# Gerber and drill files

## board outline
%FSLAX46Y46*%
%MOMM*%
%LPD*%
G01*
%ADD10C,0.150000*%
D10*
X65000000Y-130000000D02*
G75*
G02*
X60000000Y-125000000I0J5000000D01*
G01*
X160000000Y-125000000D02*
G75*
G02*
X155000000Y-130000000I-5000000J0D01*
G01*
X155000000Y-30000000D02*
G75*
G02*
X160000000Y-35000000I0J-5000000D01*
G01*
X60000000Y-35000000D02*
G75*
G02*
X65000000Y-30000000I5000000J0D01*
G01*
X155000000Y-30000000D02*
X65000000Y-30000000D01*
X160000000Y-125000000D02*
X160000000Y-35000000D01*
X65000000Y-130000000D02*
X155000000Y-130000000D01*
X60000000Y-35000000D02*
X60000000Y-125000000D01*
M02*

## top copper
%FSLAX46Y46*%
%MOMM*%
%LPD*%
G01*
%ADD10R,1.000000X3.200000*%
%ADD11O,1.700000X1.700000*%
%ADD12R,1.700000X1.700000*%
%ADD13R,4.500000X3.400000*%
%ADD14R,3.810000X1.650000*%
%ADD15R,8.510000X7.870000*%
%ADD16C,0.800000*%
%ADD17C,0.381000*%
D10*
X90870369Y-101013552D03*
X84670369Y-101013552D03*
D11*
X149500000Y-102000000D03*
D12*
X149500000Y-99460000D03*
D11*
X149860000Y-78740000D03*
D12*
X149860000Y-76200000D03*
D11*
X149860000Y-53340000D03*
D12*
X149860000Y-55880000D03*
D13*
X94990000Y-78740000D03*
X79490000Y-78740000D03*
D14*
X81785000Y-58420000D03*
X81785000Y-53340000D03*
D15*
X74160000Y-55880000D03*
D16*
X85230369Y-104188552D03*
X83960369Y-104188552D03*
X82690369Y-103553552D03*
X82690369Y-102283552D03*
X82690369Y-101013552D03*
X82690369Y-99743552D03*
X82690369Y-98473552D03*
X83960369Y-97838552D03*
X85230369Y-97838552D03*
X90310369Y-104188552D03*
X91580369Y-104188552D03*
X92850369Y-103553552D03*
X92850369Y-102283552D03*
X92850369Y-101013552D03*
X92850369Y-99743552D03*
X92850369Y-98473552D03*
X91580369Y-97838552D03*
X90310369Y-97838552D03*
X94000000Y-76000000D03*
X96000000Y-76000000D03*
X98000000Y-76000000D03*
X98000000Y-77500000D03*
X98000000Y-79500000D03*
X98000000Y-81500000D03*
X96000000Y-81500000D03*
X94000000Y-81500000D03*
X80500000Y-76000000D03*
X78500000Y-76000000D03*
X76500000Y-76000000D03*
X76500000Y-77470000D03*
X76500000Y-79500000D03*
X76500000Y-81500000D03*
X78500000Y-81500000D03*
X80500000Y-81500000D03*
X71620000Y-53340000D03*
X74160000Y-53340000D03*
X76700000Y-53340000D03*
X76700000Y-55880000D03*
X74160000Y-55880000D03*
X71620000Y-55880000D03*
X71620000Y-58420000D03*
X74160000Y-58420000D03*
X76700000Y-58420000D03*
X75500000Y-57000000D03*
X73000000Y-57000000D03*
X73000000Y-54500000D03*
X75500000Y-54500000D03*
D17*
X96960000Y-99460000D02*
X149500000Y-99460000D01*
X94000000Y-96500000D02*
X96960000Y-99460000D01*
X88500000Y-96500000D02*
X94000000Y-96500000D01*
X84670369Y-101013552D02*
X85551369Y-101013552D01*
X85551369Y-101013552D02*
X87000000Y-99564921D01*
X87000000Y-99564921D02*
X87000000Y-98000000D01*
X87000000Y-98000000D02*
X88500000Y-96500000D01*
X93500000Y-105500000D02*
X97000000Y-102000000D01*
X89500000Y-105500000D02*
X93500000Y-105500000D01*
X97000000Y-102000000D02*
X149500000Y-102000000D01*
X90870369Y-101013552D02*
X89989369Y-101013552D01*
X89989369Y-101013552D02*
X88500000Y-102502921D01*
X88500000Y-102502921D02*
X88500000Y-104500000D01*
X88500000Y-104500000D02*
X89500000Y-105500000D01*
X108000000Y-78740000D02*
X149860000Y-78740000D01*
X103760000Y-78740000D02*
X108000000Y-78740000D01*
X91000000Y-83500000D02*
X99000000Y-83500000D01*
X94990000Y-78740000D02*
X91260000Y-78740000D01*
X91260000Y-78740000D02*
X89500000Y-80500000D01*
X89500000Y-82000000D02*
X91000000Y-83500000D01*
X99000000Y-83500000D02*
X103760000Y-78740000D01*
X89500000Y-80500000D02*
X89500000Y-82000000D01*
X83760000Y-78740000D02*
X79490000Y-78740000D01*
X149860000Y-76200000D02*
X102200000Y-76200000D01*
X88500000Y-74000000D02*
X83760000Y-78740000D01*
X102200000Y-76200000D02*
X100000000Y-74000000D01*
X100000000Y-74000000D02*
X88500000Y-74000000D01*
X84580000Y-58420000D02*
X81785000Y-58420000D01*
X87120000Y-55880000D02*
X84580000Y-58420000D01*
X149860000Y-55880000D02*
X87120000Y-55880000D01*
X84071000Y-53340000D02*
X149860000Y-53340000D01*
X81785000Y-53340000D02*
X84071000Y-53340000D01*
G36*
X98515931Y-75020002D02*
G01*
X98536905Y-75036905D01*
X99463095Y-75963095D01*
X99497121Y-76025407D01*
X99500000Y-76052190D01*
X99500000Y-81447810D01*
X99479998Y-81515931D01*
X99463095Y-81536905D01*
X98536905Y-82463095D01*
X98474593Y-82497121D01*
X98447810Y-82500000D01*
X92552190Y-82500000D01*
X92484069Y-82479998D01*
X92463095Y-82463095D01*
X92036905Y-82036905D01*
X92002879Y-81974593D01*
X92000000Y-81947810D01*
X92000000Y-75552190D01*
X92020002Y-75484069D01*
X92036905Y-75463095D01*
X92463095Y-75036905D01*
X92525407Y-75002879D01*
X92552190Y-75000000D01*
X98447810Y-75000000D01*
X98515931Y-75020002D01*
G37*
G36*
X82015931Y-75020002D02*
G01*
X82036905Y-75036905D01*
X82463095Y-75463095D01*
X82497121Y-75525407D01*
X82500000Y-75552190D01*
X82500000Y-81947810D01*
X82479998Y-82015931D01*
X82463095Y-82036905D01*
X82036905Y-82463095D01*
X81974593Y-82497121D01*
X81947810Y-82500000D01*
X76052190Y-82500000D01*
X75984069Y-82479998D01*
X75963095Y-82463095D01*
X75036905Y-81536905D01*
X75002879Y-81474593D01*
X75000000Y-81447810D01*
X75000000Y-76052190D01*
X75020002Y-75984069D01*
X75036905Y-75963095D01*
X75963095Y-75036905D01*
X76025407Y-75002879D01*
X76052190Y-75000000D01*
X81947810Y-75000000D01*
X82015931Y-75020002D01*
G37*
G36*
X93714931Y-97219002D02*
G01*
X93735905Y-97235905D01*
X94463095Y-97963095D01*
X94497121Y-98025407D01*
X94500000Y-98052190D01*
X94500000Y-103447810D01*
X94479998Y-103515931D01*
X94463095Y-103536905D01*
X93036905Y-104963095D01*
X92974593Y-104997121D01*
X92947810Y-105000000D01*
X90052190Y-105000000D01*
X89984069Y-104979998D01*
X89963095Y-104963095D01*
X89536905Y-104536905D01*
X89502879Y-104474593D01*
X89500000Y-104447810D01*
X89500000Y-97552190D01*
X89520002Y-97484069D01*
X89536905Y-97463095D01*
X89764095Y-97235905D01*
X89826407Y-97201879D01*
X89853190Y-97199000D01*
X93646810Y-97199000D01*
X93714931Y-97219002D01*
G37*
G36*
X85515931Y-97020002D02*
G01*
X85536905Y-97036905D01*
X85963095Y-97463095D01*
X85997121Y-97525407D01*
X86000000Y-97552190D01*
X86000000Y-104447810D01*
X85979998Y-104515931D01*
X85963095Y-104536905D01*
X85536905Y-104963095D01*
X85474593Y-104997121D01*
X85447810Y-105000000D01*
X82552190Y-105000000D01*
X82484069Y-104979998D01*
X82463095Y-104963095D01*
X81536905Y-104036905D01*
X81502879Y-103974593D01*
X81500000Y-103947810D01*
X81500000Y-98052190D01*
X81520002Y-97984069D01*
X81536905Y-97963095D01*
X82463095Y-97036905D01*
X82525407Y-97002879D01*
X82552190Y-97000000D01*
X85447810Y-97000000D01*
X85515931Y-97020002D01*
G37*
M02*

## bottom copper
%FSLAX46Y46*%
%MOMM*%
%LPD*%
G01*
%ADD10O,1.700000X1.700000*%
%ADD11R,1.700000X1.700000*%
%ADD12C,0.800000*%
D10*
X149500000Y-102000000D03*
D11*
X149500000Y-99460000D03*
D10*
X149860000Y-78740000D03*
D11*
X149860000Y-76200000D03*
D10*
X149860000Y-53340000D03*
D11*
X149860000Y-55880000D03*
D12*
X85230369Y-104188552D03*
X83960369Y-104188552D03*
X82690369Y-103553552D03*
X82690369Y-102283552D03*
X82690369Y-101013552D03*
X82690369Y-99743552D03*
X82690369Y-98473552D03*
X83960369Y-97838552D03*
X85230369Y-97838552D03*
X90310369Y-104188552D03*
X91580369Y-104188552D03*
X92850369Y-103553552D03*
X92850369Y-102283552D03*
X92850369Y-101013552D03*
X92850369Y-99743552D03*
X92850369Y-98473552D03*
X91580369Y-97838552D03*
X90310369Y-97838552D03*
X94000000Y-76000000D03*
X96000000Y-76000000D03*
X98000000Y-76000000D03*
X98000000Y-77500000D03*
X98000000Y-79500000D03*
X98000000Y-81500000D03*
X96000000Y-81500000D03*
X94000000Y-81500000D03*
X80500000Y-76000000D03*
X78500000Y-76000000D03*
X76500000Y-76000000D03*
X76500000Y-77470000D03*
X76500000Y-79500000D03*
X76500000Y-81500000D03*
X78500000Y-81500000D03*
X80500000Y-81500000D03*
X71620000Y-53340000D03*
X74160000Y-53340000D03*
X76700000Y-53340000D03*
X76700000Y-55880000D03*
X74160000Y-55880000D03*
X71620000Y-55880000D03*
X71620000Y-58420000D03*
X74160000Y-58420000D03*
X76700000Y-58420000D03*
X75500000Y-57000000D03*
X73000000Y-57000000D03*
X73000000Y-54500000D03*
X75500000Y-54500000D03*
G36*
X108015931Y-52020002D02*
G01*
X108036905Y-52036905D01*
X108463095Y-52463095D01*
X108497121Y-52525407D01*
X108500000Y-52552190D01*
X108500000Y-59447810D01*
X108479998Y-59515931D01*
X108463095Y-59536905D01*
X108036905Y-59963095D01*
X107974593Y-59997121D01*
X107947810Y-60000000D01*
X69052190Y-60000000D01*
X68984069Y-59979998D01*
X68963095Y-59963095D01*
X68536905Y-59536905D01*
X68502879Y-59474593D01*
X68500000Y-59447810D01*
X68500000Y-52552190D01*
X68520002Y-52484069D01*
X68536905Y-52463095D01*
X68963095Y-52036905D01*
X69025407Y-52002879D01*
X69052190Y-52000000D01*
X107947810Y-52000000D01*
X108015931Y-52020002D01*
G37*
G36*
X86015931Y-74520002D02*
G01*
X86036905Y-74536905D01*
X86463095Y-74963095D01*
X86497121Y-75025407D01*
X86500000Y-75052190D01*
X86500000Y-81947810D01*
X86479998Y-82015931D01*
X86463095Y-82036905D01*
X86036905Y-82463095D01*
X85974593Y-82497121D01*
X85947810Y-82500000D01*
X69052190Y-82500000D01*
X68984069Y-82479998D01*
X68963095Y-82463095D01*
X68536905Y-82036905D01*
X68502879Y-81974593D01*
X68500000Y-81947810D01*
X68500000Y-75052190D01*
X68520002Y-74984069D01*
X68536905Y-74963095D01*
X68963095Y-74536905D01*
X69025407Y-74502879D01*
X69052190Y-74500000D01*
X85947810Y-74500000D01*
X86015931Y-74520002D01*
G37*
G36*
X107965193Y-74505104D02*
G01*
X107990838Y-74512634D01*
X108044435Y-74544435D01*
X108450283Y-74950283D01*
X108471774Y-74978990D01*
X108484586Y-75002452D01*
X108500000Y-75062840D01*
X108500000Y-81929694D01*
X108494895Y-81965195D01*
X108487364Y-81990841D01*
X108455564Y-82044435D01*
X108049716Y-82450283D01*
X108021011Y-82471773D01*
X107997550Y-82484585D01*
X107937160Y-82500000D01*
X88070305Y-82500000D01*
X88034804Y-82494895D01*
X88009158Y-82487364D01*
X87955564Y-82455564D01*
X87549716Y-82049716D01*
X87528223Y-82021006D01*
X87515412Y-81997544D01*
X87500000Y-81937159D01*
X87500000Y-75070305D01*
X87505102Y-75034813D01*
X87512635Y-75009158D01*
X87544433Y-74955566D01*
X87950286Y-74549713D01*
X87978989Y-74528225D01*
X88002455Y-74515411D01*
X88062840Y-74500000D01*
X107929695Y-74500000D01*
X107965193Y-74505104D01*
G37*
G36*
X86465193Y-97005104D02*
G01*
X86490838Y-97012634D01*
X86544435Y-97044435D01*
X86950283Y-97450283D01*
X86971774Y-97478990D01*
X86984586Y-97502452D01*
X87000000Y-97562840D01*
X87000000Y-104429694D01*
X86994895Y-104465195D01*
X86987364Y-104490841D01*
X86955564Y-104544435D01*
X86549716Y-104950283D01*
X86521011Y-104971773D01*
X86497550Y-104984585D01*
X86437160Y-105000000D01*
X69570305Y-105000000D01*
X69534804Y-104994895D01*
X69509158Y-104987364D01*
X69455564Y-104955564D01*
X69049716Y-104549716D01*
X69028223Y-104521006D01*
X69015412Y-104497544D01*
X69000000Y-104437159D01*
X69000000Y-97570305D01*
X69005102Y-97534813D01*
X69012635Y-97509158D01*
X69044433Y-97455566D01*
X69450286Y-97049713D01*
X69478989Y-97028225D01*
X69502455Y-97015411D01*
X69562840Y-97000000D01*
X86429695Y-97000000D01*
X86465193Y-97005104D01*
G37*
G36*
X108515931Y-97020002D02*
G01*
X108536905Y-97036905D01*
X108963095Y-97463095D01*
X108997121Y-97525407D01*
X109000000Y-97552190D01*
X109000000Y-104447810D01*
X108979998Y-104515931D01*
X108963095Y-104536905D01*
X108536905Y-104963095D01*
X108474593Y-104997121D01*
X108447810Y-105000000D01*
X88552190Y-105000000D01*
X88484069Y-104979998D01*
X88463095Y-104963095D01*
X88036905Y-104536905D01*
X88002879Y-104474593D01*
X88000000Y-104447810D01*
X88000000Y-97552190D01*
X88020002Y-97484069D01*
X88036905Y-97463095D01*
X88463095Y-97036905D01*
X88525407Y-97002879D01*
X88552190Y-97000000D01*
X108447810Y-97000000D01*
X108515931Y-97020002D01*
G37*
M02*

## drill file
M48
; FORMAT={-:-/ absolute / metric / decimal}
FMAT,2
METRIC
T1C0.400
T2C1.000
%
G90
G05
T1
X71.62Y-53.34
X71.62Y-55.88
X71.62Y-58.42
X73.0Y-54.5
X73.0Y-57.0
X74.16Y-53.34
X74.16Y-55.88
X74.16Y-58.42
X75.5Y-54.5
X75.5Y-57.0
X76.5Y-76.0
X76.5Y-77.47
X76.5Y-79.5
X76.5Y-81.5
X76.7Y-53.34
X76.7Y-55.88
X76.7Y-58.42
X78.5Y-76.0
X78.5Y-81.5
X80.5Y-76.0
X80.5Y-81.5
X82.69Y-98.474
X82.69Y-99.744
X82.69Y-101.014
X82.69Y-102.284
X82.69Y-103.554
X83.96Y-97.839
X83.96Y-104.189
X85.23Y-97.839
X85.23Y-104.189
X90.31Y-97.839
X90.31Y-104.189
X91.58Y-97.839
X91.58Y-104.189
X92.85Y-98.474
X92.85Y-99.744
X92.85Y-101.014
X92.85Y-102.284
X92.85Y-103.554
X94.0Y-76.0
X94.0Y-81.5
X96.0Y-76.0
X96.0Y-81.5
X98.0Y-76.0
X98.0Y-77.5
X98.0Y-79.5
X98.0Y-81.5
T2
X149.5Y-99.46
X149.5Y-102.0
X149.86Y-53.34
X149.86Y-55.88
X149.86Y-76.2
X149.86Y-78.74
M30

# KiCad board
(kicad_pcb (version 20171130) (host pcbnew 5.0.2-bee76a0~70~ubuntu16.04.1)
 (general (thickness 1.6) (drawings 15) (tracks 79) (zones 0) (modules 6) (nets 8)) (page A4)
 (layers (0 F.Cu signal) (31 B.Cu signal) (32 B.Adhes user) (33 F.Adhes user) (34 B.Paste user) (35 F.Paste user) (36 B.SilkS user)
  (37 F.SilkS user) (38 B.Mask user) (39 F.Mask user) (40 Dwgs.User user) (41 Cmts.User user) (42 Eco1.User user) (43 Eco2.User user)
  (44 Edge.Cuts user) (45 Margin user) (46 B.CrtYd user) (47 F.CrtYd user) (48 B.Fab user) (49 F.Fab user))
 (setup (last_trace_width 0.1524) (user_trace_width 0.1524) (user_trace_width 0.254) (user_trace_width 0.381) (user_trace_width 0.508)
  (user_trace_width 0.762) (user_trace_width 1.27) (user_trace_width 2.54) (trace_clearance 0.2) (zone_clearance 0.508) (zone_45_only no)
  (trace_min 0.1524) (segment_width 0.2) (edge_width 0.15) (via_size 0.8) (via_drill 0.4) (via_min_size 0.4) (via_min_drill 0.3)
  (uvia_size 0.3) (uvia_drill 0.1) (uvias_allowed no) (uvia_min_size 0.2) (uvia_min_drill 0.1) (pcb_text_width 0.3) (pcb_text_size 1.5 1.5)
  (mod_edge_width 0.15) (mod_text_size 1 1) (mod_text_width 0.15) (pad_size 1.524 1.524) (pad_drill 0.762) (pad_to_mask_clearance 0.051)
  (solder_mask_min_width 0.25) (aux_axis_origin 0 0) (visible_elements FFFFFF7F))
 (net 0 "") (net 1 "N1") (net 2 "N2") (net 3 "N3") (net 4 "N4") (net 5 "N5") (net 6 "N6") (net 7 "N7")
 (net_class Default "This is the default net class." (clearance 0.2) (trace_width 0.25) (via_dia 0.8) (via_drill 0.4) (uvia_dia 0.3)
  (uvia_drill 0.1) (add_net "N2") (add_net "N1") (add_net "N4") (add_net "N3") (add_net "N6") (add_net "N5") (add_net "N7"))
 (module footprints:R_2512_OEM (layer F.Cu) (at 87.770369 101.013552)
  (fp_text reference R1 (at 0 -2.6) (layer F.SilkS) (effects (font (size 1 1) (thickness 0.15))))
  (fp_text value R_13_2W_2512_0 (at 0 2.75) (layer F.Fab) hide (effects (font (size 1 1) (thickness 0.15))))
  (pad 2 smd rect (at 3.1 0) (size 1 3.2) (layers F.Cu F.Paste F.Mask) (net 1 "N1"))
  (pad 1 smd rect (at -3.1 0) (size 1 3.2) (layers F.Cu F.Paste F.Mask) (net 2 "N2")))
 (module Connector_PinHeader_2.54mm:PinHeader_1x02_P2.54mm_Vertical (layer F.Cu) (at 149.5 99.46)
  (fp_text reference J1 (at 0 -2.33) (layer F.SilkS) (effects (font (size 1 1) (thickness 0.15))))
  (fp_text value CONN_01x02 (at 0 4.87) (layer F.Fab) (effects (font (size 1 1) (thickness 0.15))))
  (pad 2 thru_hole oval (at 0 2.54) (size 1.7 1.7) (drill 1) (layers *.Cu *.Mask) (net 1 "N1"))
  (pad 1 thru_hole rect (at 0 0) (size 1.7 1.7) (drill 1) (layers *.Cu *.Mask) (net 2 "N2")))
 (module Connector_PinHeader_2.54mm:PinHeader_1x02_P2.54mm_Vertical (layer F.Cu) (at 149.86 76.2)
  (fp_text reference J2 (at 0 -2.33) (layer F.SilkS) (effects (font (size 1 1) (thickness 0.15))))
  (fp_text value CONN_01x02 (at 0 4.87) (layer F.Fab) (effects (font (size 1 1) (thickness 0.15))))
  (pad 2 thru_hole oval (at 0 2.54) (size 1.7 1.7) (drill 1) (layers *.Cu *.Mask) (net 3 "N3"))
  (pad 1 thru_hole rect (at 0 0) (size 1.7 1.7) (drill 1) (layers *.Cu *.Mask) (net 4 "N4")))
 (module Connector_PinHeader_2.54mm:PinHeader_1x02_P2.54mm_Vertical (layer F.Cu) (at 149.86 55.88 180)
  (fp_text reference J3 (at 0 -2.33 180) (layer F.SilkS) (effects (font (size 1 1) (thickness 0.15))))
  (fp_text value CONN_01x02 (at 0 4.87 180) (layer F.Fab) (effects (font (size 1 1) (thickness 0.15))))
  (pad 2 thru_hole oval (at 0 2.54 180) (size 1.7 1.7) (drill 1) (layers *.Cu *.Mask) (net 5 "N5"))
  (pad 1 thru_hole rect (at 0 0 180) (size 1.7 1.7) (drill 1) (layers *.Cu *.Mask) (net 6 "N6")))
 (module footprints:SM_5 (layer F.Cu) (at 87.24 78.74)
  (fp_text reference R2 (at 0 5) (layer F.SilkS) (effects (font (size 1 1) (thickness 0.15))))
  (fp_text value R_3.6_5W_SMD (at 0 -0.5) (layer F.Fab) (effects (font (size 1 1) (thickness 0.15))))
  (pad 2 smd rect (at 7.75 0) (size 4.5 3.4) (layers F.Cu F.Paste F.Mask) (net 3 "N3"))
  (pad 1 smd rect (at -7.75 0) (size 4.5 3.4) (layers F.Cu F.Paste F.Mask) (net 4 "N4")))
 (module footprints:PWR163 (layer F.Cu) (at 74.16 55.88 90)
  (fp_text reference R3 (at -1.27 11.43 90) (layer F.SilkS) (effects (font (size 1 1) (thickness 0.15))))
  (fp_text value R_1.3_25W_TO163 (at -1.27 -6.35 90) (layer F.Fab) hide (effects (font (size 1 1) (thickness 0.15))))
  (pad 1 smd rect (at -2.54 7.625 90) (size 1.65 3.81) (layers F.Cu F.Paste F.Mask) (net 6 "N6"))
  (pad 2 smd rect (at 2.54 7.625 90) (size 1.65 3.81) (layers F.Cu F.Paste F.Mask) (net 5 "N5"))
  (pad EP smd rect (at 0 0 90) (size 7.87 8.51) (layers F.Cu F.Paste F.Mask) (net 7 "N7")))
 (gr_arc (start 65 125) (end 60 125) (angle -90) (layer Edge.Cuts) (width 0.15))
 (gr_arc (start 155 125) (end 155 130) (angle -90) (layer Edge.Cuts) (width 0.15))
 (gr_arc (start 155 35) (end 160 35) (angle -90) (layer Edge.Cuts) (width 0.15))
 (gr_arc (start 65 35) (end 65 30) (angle -90) (layer Edge.Cuts) (width 0.15))
 (gr_line (start 155 30) (end 65 30) (layer Edge.Cuts) (width 0.15))
 (gr_line (start 160 125) (end 160 35) (layer Edge.Cuts) (width 0.15))
 (gr_line (start 65 130) (end 155 130) (layer Edge.Cuts) (width 0.15))
 (gr_line (start 60 35) (end 60 125) (layer Edge.Cuts) (width 0.15))
 (via (at 85.230369 104.188552) (size 0.8) (drill 0.4) (layers F.Cu B.Cu) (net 2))
 (via (at 83.960369 104.188552) (size 0.8) (drill 0.4) (layers F.Cu B.Cu) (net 2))
 (via (at 82.690369 103.553552) (size 0.8) (drill 0.4) (layers F.Cu B.Cu) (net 2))
 (via (at 82.690369 102.283552) (size 0.8) (drill 0.4) (layers F.Cu B.Cu) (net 2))
 (via (at 82.690369 101.013552) (size 0.8) (drill 0.4) (layers F.Cu B.Cu) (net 2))
 (via (at 82.690369 99.743552) (size 0.8) (drill 0.4) (layers F.Cu B.Cu) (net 2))
 (via (at 82.690369 98.473552) (size 0.8) (drill 0.4) (layers F.Cu B.Cu) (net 2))
 (via (at 83.960369 97.838552) (size 0.8) (drill 0.4) (layers F.Cu B.Cu) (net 2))
 (via (at 85.230369 97.838552) (size 0.8) (drill 0.4) (layers F.Cu B.Cu) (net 2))
 (segment (start 96.96 99.46) (end 149.5 99.46) (width 0.381) (layer F.Cu) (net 2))
 (segment (start 94 96.5) (end 96.96 99.46) (width 0.381) (layer F.Cu) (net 2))
 (segment (start 88.5 96.5) (end 94 96.5) (width 0.381) (layer F.Cu) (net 2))
 (segment (start 84.670369 101.013552) (end 85.551369 101.013552) (width 0.381) (layer F.Cu) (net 2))
 (segment (start 85.551369 101.013552) (end 87 99.564921) (width 0.381) (layer F.Cu) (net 2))
 (segment (start 87 99.564921) (end 87 98) (width 0.381) (layer F.Cu) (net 2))
 (segment (start 87 98) (end 88.5 96.5) (width 0.381) (layer F.Cu) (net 2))
 (via (at 90.310369 104.188552) (size 0.8) (drill 0.4) (layers F.Cu B.Cu) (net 1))
 (via (at 91.580369 104.188552) (size 0.8) (drill 0.4) (layers F.Cu B.Cu) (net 1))
 (via (at 92.850369 103.553552) (size 0.8) (drill 0.4) (layers F.Cu B.Cu) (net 1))
 (via (at 92.850369 102.283552) (size 0.8) (drill 0.4) (layers F.Cu B.Cu) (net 1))
 (via (at 92.850369 101.013552) (size 0.8) (drill 0.4) (layers F.Cu B.Cu) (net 1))
 (via (at 92.850369 99.743552) (size 0.8) (drill 0.4) (layers F.Cu B.Cu) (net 1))
 (via (at 92.850369 98.473552) (size 0.8) (drill 0.4) (layers F.Cu B.Cu) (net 1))
 (via (at 91.580369 97.838552) (size 0.8) (drill 0.4) (layers F.Cu B.Cu) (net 1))
 (via (at 90.310369 97.838552) (size 0.8) (drill 0.4) (layers F.Cu B.Cu) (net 1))
 (segment (start 93.5 105.5) (end 97 102) (width 0.381) (layer F.Cu) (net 1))
 (segment (start 89.5 105.5) (end 93.5 105.5) (width 0.381) (layer F.Cu) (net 1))
 (segment (start 97 102) (end 149.5 102) (width 0.381) (layer F.Cu) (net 1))
 (segment (start 90.870369 101.013552) (end 89.989369 101.013552) (width 0.381) (layer F.Cu) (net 1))
 (segment (start 89.989369 101.013552) (end 88.5 102.502921) (width 0.381) (layer F.Cu) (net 1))
 (segment (start 88.5 102.502921) (end 88.5 104.5) (width 0.381) (layer F.Cu) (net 1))
 (segment (start 88.5 104.5) (end 89.5 105.5) (width 0.381) (layer F.Cu) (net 1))
 (via (at 94 76) (size 0.8) (drill 0.4) (layers F.Cu B.Cu) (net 3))
 (via (at 96 76) (size 0.8) (drill 0.4) (layers F.Cu B.Cu) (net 3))
 (via (at 98 76) (size 0.8) (drill 0.4) (layers F.Cu B.Cu) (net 3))
 (via (at 98 77.5) (size 0.8) (drill 0.4) (layers F.Cu B.Cu) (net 3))
 (via (at 98 79.5) (size 0.8) (drill 0.4) (layers F.Cu B.Cu) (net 3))
 (via (at 98 81.5) (size 0.8) (drill 0.4) (layers F.Cu B.Cu) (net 3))
 (via (at 96 81.5) (size 0.8) (drill 0.4) (layers F.Cu B.Cu) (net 3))
 (via (at 94 81.5) (size 0.8) (drill 0.4) (layers F.Cu B.Cu) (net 3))
 (segment (start 108 78.74) (end 149.86 78.74) (width 0.381) (layer F.Cu) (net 3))
 (segment (start 103.76 78.74) (end 108 78.74) (width 0.381) (layer F.Cu) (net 3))
 (segment (start 91 83.5) (end 99 83.5) (width 0.381) (layer F.Cu) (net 3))
 (segment (start 94.99 78.74) (end 91.26 78.74) (width 0.381) (layer F.Cu) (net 3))
 (segment (start 91.26 78.74) (end 89.5 80.5) (width 0.381) (layer F.Cu) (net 3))
 (segment (start 89.5 82) (end 91 83.5) (width 0.381) (layer F.Cu) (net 3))
 (segment (start 99 83.5) (end 103.76 78.74) (width 0.381) (layer F.Cu) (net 3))
 (segment (start 89.5 80.5) (end 89.5 82) (width 0.381) (layer F.Cu) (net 3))
 (via (at 80.5 76) (size 0.8) (drill 0.4) (layers F.Cu B.Cu) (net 4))
 (via (at 78.5 76) (size 0.8) (drill 0.4) (layers F.Cu B.Cu) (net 4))
 (via (at 76.5 76) (size 0.8) (drill 0.4) (layers F.Cu B.Cu) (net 4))
 (via (at 76.5 77.47) (size 0.8) (drill 0.4) (layers F.Cu B.Cu) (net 4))
 (via (at 76.5 79.5) (size 0.8) (drill 0.4) (layers F.Cu B.Cu) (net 4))
 (via (at 76.5 81.5) (size 0.8) (drill 0.4) (layers F.Cu B.Cu) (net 4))
 (via (at 78.5 81.5) (size 0.8) (drill 0.4) (layers F.Cu B.Cu) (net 4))
 (via (at 80.5 81.5) (size 0.8) (drill 0.4) (layers F.Cu B.Cu) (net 4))
 (segment (start 83.76 78.74) (end 79.49 78.74) (width 0.381) (layer F.Cu) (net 4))
 (segment (start 149.86 76.2) (end 102.2 76.2) (width 0.381) (layer F.Cu) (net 4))
 (segment (start 88.5 74) (end 83.76 78.74) (width 0.381) (layer F.Cu) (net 4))
 (segment (start 102.2 76.2) (end 100 74) (width 0.381) (layer F.Cu) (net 4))
 (segment (start 100 74) (end 88.5 74) (width 0.381) (layer F.Cu) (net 4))
 (segment (start 84.58 58.42) (end 81.785 58.42) (width 0.381) (layer F.Cu) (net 6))
 (segment (start 87.12 55.88) (end 84.58 58.42) (width 0.381) (layer F.Cu) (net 6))
 (segment (start 149.86 55.88) (end 87.12 55.88) (width 0.381) (layer F.Cu) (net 6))
 (segment (start 84.071 53.34) (end 149.86 53.34) (width 0.381) (layer F.Cu) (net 5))
 (segment (start 81.785 53.34) (end 84.071 53.34) (width 0.381) (layer F.Cu) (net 5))
 (via (at 71.62 53.34) (size 0.8) (drill 0.4) (layers F.Cu B.Cu) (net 7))
 (via (at 74.16 53.34) (size 0.8) (drill 0.4) (layers F.Cu B.Cu) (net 7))
 (via (at 76.7 53.34) (size 0.8) (drill 0.4) (layers F.Cu B.Cu) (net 7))
 (via (at 76.7 55.88) (size 0.8) (drill 0.4) (layers F.Cu B.Cu) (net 7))
 (via (at 74.16 55.88) (size 0.8) (drill 0.4) (layers F.Cu B.Cu) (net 7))
 (via (at 71.62 55.88) (size 0.8) (drill 0.4) (layers F.Cu B.Cu) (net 7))
 (via (at 71.62 58.42) (size 0.8) (drill 0.4) (layers F.Cu B.Cu) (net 7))
 (via (at 74.16 58.42) (size 0.8) (drill 0.4) (layers F.Cu B.Cu) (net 7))
 (via (at 76.7 58.42) (size 0.8) (drill 0.4) (layers F.Cu B.Cu) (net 7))
 (via (at 75.5 57) (size 0.8) (drill 0.4) (layers F.Cu B.Cu) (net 7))
 (via (at 73 57) (size 0.8) (drill 0.4) (layers F.Cu B.Cu) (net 7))
 (via (at 73 54.5) (size 0.8) (drill 0.4) (layers F.Cu B.Cu) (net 7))
 (via (at 75.5 54.5) (size 0.8) (drill 0.4) (layers F.Cu B.Cu) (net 7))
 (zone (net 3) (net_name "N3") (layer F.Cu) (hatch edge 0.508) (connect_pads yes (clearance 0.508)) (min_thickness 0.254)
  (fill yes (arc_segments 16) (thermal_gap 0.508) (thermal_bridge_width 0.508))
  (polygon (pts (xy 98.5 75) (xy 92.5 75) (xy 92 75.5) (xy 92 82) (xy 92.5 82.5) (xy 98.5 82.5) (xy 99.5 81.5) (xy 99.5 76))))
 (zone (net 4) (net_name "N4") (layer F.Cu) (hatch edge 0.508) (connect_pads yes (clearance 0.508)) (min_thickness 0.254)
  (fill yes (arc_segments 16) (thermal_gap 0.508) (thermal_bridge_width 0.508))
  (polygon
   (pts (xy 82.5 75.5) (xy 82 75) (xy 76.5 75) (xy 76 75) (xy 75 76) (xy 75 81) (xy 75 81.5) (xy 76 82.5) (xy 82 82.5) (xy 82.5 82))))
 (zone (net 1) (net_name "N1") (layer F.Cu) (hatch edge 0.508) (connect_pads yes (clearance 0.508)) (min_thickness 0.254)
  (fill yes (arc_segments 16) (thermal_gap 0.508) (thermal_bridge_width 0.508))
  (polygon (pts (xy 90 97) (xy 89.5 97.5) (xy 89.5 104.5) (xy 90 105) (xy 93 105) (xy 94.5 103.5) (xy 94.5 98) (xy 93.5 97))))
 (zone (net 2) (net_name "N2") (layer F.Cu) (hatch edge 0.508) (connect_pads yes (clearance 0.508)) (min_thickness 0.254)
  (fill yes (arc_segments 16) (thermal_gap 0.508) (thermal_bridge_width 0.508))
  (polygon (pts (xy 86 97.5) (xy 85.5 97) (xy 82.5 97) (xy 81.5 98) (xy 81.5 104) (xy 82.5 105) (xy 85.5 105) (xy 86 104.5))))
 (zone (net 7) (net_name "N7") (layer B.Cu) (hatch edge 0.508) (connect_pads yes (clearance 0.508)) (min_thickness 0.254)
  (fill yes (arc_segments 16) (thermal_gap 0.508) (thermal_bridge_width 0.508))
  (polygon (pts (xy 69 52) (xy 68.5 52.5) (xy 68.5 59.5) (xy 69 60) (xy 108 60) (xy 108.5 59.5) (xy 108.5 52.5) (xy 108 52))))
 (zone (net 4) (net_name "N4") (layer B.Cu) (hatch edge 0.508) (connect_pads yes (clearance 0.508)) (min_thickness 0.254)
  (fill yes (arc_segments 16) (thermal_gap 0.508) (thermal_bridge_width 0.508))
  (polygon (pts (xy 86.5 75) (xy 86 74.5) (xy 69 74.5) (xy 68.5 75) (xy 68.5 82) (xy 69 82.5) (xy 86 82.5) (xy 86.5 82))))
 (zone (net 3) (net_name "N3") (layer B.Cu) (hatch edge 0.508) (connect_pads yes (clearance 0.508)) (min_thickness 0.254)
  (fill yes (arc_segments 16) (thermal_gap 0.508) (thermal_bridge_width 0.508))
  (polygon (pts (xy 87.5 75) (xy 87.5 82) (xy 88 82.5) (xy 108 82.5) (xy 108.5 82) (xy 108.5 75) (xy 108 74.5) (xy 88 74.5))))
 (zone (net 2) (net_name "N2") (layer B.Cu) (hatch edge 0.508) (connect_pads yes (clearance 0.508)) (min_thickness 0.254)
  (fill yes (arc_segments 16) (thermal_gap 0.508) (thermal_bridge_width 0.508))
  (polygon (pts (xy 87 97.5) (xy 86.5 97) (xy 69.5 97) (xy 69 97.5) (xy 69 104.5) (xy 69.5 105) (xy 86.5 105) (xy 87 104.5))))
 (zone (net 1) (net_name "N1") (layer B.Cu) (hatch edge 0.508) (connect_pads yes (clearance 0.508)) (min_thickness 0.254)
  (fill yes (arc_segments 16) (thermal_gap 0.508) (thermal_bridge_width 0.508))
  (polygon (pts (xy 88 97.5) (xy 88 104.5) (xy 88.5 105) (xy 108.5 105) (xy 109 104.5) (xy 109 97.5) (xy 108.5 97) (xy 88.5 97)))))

